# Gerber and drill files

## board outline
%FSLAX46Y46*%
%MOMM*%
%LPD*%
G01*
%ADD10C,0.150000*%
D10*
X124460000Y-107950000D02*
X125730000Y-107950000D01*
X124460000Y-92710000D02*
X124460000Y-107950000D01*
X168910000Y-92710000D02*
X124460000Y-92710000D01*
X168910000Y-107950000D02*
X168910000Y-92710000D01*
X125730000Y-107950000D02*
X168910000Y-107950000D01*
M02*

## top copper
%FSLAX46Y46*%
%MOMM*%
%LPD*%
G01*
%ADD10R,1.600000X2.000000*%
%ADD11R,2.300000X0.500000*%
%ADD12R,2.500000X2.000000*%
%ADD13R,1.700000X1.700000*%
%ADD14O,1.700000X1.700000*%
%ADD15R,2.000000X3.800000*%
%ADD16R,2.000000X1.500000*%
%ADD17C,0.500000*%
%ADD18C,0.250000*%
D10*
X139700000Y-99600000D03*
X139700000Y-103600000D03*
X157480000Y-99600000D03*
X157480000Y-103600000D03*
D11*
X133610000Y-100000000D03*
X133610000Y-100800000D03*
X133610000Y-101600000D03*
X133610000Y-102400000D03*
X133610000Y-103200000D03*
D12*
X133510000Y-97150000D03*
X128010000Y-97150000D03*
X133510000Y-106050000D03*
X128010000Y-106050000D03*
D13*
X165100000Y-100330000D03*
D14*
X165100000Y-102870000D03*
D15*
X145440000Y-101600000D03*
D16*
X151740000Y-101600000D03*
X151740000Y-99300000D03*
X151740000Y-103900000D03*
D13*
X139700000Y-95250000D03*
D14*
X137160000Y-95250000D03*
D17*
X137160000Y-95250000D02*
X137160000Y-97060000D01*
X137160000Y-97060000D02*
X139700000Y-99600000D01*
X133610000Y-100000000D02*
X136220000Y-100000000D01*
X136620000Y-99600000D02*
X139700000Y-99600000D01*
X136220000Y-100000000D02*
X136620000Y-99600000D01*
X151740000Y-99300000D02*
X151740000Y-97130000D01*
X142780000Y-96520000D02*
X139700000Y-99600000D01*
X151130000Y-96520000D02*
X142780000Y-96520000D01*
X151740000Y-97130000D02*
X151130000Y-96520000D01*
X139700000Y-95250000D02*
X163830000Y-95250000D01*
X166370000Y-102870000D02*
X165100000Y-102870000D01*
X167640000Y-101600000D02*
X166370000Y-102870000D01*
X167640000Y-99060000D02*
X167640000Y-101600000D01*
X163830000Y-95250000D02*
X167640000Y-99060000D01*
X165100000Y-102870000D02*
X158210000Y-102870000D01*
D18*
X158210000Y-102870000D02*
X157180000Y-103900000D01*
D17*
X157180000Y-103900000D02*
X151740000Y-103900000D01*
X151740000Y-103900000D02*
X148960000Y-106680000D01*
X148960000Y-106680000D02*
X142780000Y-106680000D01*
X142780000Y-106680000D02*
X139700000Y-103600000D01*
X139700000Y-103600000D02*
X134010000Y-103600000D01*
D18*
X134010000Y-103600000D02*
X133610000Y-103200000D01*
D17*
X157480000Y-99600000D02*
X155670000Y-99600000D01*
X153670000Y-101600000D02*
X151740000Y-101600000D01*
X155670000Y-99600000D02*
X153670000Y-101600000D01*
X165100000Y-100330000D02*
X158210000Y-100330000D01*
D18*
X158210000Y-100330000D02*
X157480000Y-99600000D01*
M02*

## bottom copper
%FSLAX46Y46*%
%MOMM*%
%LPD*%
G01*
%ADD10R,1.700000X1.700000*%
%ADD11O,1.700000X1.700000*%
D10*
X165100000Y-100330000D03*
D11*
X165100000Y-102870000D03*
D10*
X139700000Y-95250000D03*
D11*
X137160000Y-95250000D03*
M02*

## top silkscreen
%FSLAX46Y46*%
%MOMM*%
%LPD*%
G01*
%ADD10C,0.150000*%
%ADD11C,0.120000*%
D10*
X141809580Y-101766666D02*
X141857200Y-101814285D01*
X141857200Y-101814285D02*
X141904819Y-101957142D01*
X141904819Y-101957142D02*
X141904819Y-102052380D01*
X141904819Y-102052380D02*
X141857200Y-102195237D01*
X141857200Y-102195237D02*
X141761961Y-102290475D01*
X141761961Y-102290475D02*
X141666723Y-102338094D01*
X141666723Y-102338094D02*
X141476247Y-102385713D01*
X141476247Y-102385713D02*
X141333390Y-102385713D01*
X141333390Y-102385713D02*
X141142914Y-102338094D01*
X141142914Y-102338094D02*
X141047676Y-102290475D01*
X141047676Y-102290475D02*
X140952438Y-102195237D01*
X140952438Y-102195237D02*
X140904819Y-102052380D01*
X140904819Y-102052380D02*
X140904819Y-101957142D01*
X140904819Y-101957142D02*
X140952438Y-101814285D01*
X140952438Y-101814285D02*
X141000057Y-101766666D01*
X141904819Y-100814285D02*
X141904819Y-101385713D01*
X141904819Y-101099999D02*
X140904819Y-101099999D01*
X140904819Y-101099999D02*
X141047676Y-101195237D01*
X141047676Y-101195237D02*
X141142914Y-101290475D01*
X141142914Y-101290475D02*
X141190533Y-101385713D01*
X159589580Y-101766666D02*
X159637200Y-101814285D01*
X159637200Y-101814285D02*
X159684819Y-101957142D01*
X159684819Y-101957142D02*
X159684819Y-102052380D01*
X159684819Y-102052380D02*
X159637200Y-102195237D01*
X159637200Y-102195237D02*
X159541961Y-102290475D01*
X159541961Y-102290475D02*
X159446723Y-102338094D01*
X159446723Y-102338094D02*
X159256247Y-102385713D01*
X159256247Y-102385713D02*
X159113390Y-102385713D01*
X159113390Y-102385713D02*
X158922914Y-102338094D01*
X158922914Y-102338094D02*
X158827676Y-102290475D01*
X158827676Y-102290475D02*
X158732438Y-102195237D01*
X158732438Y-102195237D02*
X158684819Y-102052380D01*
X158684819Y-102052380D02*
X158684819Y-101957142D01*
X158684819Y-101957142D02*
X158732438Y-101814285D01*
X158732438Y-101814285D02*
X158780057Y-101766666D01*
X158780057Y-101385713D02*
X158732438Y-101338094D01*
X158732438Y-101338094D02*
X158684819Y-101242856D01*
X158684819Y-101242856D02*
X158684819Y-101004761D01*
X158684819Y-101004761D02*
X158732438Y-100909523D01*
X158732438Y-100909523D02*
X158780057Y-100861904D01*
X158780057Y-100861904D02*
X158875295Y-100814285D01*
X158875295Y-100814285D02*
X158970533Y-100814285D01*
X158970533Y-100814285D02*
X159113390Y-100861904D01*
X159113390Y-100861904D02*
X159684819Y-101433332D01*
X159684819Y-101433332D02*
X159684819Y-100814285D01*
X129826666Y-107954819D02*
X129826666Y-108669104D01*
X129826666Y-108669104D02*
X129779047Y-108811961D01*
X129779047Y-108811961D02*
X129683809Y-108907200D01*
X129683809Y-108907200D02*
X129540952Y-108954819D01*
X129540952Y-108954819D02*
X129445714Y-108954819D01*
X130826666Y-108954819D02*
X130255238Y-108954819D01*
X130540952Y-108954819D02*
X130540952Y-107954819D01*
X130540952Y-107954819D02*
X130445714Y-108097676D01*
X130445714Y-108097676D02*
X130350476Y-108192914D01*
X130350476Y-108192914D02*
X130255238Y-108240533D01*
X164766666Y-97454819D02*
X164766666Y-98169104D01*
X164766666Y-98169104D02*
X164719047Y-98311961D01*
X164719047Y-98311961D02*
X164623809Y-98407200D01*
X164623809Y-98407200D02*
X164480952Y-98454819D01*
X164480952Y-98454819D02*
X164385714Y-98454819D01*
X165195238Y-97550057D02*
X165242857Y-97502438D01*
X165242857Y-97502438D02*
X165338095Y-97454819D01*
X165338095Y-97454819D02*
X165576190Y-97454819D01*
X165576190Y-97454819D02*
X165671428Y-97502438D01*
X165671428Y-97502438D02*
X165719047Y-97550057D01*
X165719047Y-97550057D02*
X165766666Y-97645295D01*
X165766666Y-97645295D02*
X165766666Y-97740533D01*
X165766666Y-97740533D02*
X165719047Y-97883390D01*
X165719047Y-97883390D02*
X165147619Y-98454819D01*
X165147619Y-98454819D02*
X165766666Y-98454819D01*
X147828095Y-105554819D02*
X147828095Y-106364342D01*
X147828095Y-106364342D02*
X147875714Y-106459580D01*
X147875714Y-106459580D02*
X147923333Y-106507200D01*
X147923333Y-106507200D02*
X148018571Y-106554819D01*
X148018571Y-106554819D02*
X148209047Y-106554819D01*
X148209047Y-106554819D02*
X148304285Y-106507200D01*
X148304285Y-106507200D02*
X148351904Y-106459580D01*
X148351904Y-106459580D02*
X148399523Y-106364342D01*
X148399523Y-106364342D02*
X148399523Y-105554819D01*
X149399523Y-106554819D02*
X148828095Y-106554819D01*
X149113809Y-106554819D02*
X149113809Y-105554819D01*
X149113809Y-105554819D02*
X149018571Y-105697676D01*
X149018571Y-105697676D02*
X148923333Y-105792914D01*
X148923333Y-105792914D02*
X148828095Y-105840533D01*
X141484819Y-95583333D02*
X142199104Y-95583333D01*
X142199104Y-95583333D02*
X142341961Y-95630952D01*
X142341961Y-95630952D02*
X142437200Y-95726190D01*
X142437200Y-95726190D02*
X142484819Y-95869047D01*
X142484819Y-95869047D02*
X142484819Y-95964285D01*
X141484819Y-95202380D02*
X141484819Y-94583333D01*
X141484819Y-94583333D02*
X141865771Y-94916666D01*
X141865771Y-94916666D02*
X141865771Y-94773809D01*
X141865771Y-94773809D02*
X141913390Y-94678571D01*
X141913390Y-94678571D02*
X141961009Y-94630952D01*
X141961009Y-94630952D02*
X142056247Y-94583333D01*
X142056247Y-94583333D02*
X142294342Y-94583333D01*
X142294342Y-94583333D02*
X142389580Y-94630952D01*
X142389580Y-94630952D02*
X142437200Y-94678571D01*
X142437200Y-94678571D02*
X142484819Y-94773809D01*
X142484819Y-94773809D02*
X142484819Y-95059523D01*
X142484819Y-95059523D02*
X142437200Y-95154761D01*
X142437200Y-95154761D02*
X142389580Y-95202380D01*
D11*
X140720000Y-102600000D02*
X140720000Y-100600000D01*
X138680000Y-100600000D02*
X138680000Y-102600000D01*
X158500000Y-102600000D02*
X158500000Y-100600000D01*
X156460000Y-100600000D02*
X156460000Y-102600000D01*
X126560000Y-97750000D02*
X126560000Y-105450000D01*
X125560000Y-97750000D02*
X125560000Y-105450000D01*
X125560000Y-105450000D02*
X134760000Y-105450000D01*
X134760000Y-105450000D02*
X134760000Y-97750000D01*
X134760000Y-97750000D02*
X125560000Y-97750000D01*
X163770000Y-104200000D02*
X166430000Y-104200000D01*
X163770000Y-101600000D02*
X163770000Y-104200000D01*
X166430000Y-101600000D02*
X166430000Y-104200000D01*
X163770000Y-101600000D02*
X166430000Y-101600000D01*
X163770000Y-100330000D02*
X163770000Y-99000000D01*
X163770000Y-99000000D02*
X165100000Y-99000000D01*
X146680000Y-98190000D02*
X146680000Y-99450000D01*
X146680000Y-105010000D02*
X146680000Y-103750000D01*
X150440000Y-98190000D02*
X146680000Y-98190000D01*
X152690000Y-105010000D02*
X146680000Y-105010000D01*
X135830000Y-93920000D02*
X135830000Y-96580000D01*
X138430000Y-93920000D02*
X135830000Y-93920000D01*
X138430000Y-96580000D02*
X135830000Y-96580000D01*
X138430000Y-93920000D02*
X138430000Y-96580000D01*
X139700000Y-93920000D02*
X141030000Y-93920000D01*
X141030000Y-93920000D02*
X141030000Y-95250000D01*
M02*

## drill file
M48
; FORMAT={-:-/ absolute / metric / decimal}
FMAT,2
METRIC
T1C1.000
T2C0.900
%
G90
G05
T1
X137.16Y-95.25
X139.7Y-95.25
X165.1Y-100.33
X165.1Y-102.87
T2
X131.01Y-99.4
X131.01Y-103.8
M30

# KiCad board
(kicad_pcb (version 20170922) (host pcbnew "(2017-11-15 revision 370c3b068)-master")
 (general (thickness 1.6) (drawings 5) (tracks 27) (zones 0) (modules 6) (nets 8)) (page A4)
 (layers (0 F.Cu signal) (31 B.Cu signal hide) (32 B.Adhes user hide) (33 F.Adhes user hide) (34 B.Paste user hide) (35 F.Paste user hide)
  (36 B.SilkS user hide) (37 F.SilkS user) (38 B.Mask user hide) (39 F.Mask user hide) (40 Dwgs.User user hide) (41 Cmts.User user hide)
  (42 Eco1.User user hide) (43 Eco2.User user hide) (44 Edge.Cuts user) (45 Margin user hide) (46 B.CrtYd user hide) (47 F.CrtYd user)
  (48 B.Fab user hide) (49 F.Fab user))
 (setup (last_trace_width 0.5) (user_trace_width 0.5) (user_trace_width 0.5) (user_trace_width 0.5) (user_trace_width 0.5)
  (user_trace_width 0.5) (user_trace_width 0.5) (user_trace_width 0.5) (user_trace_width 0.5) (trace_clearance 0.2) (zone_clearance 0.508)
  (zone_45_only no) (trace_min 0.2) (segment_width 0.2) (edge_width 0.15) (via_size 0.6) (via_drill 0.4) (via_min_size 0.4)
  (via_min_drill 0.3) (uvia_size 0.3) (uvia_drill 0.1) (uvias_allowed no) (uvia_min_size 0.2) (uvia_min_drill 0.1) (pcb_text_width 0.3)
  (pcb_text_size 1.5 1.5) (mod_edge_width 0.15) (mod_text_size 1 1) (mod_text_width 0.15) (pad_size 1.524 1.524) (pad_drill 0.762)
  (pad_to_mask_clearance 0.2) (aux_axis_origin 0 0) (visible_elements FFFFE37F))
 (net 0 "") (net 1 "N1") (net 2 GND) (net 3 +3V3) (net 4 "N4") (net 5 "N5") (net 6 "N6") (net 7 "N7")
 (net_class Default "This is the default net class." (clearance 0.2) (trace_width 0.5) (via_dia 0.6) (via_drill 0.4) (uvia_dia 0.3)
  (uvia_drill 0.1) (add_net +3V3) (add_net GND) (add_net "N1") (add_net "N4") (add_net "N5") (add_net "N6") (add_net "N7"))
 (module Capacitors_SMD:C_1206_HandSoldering (layer F.Cu) (at 139.7 101.6 270)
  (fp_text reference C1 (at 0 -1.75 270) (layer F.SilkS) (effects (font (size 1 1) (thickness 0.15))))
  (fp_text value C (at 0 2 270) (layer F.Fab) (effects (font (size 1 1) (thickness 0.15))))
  (fp_line (start 1 -1.02) (end -1 -1.02) (layer F.SilkS) (width 0.12))
  (fp_line (start -1 1.02) (end 1 1.02) (layer F.SilkS) (width 0.12))
  (pad 1 smd rect (at -2 0 270) (size 2 1.6) (layers F.Cu F.Paste F.Mask) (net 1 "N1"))
  (pad 2 smd rect (at 2 0 270) (size 2 1.6) (layers F.Cu F.Paste F.Mask) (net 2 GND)))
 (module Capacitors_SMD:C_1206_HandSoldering (layer F.Cu) (at 157.48 101.6 270)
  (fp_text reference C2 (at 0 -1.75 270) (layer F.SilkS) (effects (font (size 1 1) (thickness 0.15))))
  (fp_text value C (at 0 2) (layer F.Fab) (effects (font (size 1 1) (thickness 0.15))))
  (fp_line (start 1 -1.02) (end -1 -1.02) (layer F.SilkS) (width 0.12))
  (fp_line (start -1 1.02) (end 1 1.02) (layer F.SilkS) (width 0.12))
  (pad 1 smd rect (at -2 0 270) (size 2 1.6) (layers F.Cu F.Paste F.Mask) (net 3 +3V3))
  (pad 2 smd rect (at 2 0 270) (size 2 1.6) (layers F.Cu F.Paste F.Mask) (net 2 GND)))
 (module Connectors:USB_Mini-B (layer F.Cu) (at 130.81 101.6)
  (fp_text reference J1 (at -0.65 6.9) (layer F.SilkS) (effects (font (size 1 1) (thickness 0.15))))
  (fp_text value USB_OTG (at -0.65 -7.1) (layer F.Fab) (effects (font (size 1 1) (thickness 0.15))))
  (fp_line (start -4.25 -3.85) (end -4.25 3.85) (layer F.SilkS) (width 0.12))
  (fp_line (start -5.25 -3.85) (end -5.25 3.85) (layer F.SilkS) (width 0.12))
  (fp_line (start -5.25 3.85) (end 3.95 3.85) (layer F.SilkS) (width 0.12))
  (fp_line (start 3.95 3.85) (end 3.95 -3.85) (layer F.SilkS) (width 0.12))
  (fp_line (start 3.95 -3.85) (end -5.25 -3.85) (layer F.SilkS) (width 0.12))
  (pad 1 smd rect (at 2.8 -1.6) (size 2.3 0.5) (layers F.Cu F.Paste F.Mask) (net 1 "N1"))
  (pad 2 smd rect (at 2.8 -0.8) (size 2.3 0.5) (layers F.Cu F.Paste F.Mask) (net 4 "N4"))
  (pad 3 smd rect (at 2.8 0) (size 2.3 0.5) (layers F.Cu F.Paste F.Mask) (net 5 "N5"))
  (pad 4 smd rect (at 2.8 0.8) (size 2.3 0.5) (layers F.Cu F.Paste F.Mask) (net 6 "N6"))
  (pad 5 smd rect (at 2.8 1.6) (size 2.3 0.5) (layers F.Cu F.Paste F.Mask) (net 2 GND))
  (pad 6 smd rect (at 2.7 -4.45) (size 2.5 2) (layers F.Cu F.Paste F.Mask) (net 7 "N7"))
  (pad 6 smd rect (at -2.8 -4.45) (size 2.5 2) (layers F.Cu F.Paste F.Mask) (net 7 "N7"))
  (pad 6 smd rect (at 2.7 4.45) (size 2.5 2) (layers F.Cu F.Paste F.Mask) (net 7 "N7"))
  (pad 6 smd rect (at -2.8 4.45) (size 2.5 2) (layers F.Cu F.Paste F.Mask) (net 7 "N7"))
  (pad "" np_thru_hole circle (at 0.2 -2.2) (size 0.9 0.9) (drill 0.9) (layers *.Cu *.Mask))
  (pad "" np_thru_hole circle (at 0.2 2.2) (size 0.9 0.9) (drill 0.9) (layers *.Cu *.Mask)))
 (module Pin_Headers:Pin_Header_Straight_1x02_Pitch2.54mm (layer F.Cu) (at 165.1 100.33)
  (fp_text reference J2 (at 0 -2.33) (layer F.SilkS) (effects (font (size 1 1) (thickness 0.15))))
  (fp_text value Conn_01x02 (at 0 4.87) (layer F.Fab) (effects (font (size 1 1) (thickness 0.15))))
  (fp_line (start -1.33 3.87) (end 1.33 3.87) (layer F.SilkS) (width 0.12))
  (fp_line (start -1.33 1.27) (end -1.33 3.87) (layer F.SilkS) (width 0.12))
  (fp_line (start 1.33 1.27) (end 1.33 3.87) (layer F.SilkS) (width 0.12))
  (fp_line (start -1.33 1.27) (end 1.33 1.27) (layer F.SilkS) (width 0.12))
  (fp_line (start -1.33 0) (end -1.33 -1.33) (layer F.SilkS) (width 0.12))
  (fp_line (start -1.33 -1.33) (end 0 -1.33) (layer F.SilkS) (width 0.12))
  (pad 1 thru_hole rect (at 0 0) (size 1.7 1.7) (drill 1) (layers *.Cu *.Mask) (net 3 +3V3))
  (pad 2 thru_hole oval (at 0 2.54) (size 1.7 1.7) (drill 1) (layers *.Cu *.Mask) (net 2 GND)))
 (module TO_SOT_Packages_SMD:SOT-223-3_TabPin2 (layer F.Cu) (at 148.59 101.6 180)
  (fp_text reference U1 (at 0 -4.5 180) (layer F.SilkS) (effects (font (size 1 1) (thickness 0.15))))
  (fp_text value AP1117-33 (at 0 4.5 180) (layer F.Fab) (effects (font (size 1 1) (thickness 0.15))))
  (fp_line (start 1.91 3.41) (end 1.91 2.15) (layer F.SilkS) (width 0.12))
  (fp_line (start 1.91 -3.41) (end 1.91 -2.15) (layer F.SilkS) (width 0.12))
  (fp_line (start -1.85 3.41) (end 1.91 3.41) (layer F.SilkS) (width 0.12))
  (fp_line (start -4.1 -3.41) (end 1.91 -3.41) (layer F.SilkS) (width 0.12))
  (pad 2 smd rect (at 3.15 0 180) (size 2 3.8) (layers F.Cu F.Paste F.Mask) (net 3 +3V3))
  (pad 2 smd rect (at -3.15 0 180) (size 2 1.5) (layers F.Cu F.Paste F.Mask) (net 3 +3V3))
  (pad 3 smd rect (at -3.15 2.3 180) (size 2 1.5) (layers F.Cu F.Paste F.Mask) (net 1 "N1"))
  (pad 1 smd rect (at -3.15 -2.3 180) (size 2 1.5) (layers F.Cu F.Paste F.Mask) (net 2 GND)))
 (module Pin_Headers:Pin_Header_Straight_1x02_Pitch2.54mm (layer F.Cu) (at 139.7 95.25 270)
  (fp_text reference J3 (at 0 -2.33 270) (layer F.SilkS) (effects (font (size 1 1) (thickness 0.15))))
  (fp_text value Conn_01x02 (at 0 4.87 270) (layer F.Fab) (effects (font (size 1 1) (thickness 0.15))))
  (fp_line (start -1.33 3.87) (end 1.33 3.87) (layer F.SilkS) (width 0.12))
  (fp_line (start -1.33 1.27) (end -1.33 3.87) (layer F.SilkS) (width 0.12))
  (fp_line (start 1.33 1.27) (end 1.33 3.87) (layer F.SilkS) (width 0.12))
  (fp_line (start -1.33 1.27) (end 1.33 1.27) (layer F.SilkS) (width 0.12))
  (fp_line (start -1.33 0) (end -1.33 -1.33) (layer F.SilkS) (width 0.12))
  (fp_line (start -1.33 -1.33) (end 0 -1.33) (layer F.SilkS) (width 0.12))
  (pad 1 thru_hole rect (at 0 0 270) (size 1.7 1.7) (drill 1) (layers *.Cu *.Mask) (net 2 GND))
  (pad 2 thru_hole oval (at 0 2.54 270) (size 1.7 1.7) (drill 1) (layers *.Cu *.Mask) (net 1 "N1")))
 (gr_line (start 124.46 107.95) (end 125.73 107.95) (layer Edge.Cuts) (width 0.15))
 (gr_line (start 124.46 92.71) (end 124.46 107.95) (layer Edge.Cuts) (width 0.15))
 (gr_line (start 168.91 92.71) (end 124.46 92.71) (layer Edge.Cuts) (width 0.15))
 (gr_line (start 168.91 107.95) (end 168.91 92.71) (layer Edge.Cuts) (width 0.15))
 (gr_line (start 125.73 107.95) (end 168.91 107.95) (layer Edge.Cuts) (width 0.15))
 (segment (start 137.16 95.25) (end 137.16 97.06) (width 0.5) (layer F.Cu) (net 1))
 (segment (start 137.16 97.06) (end 139.7 99.6) (width 0.5) (layer F.Cu) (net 1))
 (segment (start 133.61 100) (end 136.22 100) (width 0.5) (layer F.Cu) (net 1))
 (segment (start 136.62 99.6) (end 139.7 99.6) (width 0.5) (layer F.Cu) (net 1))
 (segment (start 136.22 100) (end 136.62 99.6) (width 0.5) (layer F.Cu) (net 1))
 (segment (start 151.74 99.3) (end 151.74 97.13) (width 0.5) (layer F.Cu) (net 1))
 (segment (start 142.78 96.52) (end 139.7 99.6) (width 0.5) (layer F.Cu) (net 1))
 (segment (start 151.13 96.52) (end 142.78 96.52) (width 0.5) (layer F.Cu) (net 1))
 (segment (start 151.74 97.13) (end 151.13 96.52) (width 0.5) (layer F.Cu) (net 1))
 (segment (start 139.7 95.25) (end 163.83 95.25) (width 0.5) (layer F.Cu) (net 2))
 (segment (start 166.37 102.87) (end 165.1 102.87) (width 0.5) (layer F.Cu) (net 2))
 (segment (start 167.64 101.6) (end 166.37 102.87) (width 0.5) (layer F.Cu) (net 2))
 (segment (start 167.64 99.06) (end 167.64 101.6) (width 0.5) (layer F.Cu) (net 2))
 (segment (start 163.83 95.25) (end 167.64 99.06) (width 0.5) (layer F.Cu) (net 2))
 (segment (start 165.1 102.87) (end 158.21 102.87) (width 0.5) (layer F.Cu) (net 2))
 (segment (start 158.21 102.87) (end 157.18 103.9) (width 0.25) (layer F.Cu) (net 2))
 (segment (start 157.18 103.9) (end 151.74 103.9) (width 0.5) (layer F.Cu) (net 2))
 (segment (start 151.74 103.9) (end 148.96 106.68) (width 0.5) (layer F.Cu) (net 2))
 (segment (start 148.96 106.68) (end 142.78 106.68) (width 0.5) (layer F.Cu) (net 2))
 (segment (start 142.78 106.68) (end 139.7 103.6) (width 0.5) (layer F.Cu) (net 2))
 (segment (start 139.7 103.6) (end 134.01 103.6) (width 0.5) (layer F.Cu) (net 2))
 (segment (start 134.01 103.6) (end 133.61 103.2) (width 0.25) (layer F.Cu) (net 2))
 (segment (start 157.48 99.6) (end 155.67 99.6) (width 0.5) (layer F.Cu) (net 3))
 (segment (start 153.67 101.6) (end 151.74 101.6) (width 0.5) (layer F.Cu) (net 3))
 (segment (start 155.67 99.6) (end 153.67 101.6) (width 0.5) (layer F.Cu) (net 3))
 (segment (start 165.1 100.33) (end 158.21 100.33) (width 0.5) (layer F.Cu) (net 3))
 (segment (start 158.21 100.33) (end 157.48 99.6) (width 0.25) (layer F.Cu) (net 3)))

